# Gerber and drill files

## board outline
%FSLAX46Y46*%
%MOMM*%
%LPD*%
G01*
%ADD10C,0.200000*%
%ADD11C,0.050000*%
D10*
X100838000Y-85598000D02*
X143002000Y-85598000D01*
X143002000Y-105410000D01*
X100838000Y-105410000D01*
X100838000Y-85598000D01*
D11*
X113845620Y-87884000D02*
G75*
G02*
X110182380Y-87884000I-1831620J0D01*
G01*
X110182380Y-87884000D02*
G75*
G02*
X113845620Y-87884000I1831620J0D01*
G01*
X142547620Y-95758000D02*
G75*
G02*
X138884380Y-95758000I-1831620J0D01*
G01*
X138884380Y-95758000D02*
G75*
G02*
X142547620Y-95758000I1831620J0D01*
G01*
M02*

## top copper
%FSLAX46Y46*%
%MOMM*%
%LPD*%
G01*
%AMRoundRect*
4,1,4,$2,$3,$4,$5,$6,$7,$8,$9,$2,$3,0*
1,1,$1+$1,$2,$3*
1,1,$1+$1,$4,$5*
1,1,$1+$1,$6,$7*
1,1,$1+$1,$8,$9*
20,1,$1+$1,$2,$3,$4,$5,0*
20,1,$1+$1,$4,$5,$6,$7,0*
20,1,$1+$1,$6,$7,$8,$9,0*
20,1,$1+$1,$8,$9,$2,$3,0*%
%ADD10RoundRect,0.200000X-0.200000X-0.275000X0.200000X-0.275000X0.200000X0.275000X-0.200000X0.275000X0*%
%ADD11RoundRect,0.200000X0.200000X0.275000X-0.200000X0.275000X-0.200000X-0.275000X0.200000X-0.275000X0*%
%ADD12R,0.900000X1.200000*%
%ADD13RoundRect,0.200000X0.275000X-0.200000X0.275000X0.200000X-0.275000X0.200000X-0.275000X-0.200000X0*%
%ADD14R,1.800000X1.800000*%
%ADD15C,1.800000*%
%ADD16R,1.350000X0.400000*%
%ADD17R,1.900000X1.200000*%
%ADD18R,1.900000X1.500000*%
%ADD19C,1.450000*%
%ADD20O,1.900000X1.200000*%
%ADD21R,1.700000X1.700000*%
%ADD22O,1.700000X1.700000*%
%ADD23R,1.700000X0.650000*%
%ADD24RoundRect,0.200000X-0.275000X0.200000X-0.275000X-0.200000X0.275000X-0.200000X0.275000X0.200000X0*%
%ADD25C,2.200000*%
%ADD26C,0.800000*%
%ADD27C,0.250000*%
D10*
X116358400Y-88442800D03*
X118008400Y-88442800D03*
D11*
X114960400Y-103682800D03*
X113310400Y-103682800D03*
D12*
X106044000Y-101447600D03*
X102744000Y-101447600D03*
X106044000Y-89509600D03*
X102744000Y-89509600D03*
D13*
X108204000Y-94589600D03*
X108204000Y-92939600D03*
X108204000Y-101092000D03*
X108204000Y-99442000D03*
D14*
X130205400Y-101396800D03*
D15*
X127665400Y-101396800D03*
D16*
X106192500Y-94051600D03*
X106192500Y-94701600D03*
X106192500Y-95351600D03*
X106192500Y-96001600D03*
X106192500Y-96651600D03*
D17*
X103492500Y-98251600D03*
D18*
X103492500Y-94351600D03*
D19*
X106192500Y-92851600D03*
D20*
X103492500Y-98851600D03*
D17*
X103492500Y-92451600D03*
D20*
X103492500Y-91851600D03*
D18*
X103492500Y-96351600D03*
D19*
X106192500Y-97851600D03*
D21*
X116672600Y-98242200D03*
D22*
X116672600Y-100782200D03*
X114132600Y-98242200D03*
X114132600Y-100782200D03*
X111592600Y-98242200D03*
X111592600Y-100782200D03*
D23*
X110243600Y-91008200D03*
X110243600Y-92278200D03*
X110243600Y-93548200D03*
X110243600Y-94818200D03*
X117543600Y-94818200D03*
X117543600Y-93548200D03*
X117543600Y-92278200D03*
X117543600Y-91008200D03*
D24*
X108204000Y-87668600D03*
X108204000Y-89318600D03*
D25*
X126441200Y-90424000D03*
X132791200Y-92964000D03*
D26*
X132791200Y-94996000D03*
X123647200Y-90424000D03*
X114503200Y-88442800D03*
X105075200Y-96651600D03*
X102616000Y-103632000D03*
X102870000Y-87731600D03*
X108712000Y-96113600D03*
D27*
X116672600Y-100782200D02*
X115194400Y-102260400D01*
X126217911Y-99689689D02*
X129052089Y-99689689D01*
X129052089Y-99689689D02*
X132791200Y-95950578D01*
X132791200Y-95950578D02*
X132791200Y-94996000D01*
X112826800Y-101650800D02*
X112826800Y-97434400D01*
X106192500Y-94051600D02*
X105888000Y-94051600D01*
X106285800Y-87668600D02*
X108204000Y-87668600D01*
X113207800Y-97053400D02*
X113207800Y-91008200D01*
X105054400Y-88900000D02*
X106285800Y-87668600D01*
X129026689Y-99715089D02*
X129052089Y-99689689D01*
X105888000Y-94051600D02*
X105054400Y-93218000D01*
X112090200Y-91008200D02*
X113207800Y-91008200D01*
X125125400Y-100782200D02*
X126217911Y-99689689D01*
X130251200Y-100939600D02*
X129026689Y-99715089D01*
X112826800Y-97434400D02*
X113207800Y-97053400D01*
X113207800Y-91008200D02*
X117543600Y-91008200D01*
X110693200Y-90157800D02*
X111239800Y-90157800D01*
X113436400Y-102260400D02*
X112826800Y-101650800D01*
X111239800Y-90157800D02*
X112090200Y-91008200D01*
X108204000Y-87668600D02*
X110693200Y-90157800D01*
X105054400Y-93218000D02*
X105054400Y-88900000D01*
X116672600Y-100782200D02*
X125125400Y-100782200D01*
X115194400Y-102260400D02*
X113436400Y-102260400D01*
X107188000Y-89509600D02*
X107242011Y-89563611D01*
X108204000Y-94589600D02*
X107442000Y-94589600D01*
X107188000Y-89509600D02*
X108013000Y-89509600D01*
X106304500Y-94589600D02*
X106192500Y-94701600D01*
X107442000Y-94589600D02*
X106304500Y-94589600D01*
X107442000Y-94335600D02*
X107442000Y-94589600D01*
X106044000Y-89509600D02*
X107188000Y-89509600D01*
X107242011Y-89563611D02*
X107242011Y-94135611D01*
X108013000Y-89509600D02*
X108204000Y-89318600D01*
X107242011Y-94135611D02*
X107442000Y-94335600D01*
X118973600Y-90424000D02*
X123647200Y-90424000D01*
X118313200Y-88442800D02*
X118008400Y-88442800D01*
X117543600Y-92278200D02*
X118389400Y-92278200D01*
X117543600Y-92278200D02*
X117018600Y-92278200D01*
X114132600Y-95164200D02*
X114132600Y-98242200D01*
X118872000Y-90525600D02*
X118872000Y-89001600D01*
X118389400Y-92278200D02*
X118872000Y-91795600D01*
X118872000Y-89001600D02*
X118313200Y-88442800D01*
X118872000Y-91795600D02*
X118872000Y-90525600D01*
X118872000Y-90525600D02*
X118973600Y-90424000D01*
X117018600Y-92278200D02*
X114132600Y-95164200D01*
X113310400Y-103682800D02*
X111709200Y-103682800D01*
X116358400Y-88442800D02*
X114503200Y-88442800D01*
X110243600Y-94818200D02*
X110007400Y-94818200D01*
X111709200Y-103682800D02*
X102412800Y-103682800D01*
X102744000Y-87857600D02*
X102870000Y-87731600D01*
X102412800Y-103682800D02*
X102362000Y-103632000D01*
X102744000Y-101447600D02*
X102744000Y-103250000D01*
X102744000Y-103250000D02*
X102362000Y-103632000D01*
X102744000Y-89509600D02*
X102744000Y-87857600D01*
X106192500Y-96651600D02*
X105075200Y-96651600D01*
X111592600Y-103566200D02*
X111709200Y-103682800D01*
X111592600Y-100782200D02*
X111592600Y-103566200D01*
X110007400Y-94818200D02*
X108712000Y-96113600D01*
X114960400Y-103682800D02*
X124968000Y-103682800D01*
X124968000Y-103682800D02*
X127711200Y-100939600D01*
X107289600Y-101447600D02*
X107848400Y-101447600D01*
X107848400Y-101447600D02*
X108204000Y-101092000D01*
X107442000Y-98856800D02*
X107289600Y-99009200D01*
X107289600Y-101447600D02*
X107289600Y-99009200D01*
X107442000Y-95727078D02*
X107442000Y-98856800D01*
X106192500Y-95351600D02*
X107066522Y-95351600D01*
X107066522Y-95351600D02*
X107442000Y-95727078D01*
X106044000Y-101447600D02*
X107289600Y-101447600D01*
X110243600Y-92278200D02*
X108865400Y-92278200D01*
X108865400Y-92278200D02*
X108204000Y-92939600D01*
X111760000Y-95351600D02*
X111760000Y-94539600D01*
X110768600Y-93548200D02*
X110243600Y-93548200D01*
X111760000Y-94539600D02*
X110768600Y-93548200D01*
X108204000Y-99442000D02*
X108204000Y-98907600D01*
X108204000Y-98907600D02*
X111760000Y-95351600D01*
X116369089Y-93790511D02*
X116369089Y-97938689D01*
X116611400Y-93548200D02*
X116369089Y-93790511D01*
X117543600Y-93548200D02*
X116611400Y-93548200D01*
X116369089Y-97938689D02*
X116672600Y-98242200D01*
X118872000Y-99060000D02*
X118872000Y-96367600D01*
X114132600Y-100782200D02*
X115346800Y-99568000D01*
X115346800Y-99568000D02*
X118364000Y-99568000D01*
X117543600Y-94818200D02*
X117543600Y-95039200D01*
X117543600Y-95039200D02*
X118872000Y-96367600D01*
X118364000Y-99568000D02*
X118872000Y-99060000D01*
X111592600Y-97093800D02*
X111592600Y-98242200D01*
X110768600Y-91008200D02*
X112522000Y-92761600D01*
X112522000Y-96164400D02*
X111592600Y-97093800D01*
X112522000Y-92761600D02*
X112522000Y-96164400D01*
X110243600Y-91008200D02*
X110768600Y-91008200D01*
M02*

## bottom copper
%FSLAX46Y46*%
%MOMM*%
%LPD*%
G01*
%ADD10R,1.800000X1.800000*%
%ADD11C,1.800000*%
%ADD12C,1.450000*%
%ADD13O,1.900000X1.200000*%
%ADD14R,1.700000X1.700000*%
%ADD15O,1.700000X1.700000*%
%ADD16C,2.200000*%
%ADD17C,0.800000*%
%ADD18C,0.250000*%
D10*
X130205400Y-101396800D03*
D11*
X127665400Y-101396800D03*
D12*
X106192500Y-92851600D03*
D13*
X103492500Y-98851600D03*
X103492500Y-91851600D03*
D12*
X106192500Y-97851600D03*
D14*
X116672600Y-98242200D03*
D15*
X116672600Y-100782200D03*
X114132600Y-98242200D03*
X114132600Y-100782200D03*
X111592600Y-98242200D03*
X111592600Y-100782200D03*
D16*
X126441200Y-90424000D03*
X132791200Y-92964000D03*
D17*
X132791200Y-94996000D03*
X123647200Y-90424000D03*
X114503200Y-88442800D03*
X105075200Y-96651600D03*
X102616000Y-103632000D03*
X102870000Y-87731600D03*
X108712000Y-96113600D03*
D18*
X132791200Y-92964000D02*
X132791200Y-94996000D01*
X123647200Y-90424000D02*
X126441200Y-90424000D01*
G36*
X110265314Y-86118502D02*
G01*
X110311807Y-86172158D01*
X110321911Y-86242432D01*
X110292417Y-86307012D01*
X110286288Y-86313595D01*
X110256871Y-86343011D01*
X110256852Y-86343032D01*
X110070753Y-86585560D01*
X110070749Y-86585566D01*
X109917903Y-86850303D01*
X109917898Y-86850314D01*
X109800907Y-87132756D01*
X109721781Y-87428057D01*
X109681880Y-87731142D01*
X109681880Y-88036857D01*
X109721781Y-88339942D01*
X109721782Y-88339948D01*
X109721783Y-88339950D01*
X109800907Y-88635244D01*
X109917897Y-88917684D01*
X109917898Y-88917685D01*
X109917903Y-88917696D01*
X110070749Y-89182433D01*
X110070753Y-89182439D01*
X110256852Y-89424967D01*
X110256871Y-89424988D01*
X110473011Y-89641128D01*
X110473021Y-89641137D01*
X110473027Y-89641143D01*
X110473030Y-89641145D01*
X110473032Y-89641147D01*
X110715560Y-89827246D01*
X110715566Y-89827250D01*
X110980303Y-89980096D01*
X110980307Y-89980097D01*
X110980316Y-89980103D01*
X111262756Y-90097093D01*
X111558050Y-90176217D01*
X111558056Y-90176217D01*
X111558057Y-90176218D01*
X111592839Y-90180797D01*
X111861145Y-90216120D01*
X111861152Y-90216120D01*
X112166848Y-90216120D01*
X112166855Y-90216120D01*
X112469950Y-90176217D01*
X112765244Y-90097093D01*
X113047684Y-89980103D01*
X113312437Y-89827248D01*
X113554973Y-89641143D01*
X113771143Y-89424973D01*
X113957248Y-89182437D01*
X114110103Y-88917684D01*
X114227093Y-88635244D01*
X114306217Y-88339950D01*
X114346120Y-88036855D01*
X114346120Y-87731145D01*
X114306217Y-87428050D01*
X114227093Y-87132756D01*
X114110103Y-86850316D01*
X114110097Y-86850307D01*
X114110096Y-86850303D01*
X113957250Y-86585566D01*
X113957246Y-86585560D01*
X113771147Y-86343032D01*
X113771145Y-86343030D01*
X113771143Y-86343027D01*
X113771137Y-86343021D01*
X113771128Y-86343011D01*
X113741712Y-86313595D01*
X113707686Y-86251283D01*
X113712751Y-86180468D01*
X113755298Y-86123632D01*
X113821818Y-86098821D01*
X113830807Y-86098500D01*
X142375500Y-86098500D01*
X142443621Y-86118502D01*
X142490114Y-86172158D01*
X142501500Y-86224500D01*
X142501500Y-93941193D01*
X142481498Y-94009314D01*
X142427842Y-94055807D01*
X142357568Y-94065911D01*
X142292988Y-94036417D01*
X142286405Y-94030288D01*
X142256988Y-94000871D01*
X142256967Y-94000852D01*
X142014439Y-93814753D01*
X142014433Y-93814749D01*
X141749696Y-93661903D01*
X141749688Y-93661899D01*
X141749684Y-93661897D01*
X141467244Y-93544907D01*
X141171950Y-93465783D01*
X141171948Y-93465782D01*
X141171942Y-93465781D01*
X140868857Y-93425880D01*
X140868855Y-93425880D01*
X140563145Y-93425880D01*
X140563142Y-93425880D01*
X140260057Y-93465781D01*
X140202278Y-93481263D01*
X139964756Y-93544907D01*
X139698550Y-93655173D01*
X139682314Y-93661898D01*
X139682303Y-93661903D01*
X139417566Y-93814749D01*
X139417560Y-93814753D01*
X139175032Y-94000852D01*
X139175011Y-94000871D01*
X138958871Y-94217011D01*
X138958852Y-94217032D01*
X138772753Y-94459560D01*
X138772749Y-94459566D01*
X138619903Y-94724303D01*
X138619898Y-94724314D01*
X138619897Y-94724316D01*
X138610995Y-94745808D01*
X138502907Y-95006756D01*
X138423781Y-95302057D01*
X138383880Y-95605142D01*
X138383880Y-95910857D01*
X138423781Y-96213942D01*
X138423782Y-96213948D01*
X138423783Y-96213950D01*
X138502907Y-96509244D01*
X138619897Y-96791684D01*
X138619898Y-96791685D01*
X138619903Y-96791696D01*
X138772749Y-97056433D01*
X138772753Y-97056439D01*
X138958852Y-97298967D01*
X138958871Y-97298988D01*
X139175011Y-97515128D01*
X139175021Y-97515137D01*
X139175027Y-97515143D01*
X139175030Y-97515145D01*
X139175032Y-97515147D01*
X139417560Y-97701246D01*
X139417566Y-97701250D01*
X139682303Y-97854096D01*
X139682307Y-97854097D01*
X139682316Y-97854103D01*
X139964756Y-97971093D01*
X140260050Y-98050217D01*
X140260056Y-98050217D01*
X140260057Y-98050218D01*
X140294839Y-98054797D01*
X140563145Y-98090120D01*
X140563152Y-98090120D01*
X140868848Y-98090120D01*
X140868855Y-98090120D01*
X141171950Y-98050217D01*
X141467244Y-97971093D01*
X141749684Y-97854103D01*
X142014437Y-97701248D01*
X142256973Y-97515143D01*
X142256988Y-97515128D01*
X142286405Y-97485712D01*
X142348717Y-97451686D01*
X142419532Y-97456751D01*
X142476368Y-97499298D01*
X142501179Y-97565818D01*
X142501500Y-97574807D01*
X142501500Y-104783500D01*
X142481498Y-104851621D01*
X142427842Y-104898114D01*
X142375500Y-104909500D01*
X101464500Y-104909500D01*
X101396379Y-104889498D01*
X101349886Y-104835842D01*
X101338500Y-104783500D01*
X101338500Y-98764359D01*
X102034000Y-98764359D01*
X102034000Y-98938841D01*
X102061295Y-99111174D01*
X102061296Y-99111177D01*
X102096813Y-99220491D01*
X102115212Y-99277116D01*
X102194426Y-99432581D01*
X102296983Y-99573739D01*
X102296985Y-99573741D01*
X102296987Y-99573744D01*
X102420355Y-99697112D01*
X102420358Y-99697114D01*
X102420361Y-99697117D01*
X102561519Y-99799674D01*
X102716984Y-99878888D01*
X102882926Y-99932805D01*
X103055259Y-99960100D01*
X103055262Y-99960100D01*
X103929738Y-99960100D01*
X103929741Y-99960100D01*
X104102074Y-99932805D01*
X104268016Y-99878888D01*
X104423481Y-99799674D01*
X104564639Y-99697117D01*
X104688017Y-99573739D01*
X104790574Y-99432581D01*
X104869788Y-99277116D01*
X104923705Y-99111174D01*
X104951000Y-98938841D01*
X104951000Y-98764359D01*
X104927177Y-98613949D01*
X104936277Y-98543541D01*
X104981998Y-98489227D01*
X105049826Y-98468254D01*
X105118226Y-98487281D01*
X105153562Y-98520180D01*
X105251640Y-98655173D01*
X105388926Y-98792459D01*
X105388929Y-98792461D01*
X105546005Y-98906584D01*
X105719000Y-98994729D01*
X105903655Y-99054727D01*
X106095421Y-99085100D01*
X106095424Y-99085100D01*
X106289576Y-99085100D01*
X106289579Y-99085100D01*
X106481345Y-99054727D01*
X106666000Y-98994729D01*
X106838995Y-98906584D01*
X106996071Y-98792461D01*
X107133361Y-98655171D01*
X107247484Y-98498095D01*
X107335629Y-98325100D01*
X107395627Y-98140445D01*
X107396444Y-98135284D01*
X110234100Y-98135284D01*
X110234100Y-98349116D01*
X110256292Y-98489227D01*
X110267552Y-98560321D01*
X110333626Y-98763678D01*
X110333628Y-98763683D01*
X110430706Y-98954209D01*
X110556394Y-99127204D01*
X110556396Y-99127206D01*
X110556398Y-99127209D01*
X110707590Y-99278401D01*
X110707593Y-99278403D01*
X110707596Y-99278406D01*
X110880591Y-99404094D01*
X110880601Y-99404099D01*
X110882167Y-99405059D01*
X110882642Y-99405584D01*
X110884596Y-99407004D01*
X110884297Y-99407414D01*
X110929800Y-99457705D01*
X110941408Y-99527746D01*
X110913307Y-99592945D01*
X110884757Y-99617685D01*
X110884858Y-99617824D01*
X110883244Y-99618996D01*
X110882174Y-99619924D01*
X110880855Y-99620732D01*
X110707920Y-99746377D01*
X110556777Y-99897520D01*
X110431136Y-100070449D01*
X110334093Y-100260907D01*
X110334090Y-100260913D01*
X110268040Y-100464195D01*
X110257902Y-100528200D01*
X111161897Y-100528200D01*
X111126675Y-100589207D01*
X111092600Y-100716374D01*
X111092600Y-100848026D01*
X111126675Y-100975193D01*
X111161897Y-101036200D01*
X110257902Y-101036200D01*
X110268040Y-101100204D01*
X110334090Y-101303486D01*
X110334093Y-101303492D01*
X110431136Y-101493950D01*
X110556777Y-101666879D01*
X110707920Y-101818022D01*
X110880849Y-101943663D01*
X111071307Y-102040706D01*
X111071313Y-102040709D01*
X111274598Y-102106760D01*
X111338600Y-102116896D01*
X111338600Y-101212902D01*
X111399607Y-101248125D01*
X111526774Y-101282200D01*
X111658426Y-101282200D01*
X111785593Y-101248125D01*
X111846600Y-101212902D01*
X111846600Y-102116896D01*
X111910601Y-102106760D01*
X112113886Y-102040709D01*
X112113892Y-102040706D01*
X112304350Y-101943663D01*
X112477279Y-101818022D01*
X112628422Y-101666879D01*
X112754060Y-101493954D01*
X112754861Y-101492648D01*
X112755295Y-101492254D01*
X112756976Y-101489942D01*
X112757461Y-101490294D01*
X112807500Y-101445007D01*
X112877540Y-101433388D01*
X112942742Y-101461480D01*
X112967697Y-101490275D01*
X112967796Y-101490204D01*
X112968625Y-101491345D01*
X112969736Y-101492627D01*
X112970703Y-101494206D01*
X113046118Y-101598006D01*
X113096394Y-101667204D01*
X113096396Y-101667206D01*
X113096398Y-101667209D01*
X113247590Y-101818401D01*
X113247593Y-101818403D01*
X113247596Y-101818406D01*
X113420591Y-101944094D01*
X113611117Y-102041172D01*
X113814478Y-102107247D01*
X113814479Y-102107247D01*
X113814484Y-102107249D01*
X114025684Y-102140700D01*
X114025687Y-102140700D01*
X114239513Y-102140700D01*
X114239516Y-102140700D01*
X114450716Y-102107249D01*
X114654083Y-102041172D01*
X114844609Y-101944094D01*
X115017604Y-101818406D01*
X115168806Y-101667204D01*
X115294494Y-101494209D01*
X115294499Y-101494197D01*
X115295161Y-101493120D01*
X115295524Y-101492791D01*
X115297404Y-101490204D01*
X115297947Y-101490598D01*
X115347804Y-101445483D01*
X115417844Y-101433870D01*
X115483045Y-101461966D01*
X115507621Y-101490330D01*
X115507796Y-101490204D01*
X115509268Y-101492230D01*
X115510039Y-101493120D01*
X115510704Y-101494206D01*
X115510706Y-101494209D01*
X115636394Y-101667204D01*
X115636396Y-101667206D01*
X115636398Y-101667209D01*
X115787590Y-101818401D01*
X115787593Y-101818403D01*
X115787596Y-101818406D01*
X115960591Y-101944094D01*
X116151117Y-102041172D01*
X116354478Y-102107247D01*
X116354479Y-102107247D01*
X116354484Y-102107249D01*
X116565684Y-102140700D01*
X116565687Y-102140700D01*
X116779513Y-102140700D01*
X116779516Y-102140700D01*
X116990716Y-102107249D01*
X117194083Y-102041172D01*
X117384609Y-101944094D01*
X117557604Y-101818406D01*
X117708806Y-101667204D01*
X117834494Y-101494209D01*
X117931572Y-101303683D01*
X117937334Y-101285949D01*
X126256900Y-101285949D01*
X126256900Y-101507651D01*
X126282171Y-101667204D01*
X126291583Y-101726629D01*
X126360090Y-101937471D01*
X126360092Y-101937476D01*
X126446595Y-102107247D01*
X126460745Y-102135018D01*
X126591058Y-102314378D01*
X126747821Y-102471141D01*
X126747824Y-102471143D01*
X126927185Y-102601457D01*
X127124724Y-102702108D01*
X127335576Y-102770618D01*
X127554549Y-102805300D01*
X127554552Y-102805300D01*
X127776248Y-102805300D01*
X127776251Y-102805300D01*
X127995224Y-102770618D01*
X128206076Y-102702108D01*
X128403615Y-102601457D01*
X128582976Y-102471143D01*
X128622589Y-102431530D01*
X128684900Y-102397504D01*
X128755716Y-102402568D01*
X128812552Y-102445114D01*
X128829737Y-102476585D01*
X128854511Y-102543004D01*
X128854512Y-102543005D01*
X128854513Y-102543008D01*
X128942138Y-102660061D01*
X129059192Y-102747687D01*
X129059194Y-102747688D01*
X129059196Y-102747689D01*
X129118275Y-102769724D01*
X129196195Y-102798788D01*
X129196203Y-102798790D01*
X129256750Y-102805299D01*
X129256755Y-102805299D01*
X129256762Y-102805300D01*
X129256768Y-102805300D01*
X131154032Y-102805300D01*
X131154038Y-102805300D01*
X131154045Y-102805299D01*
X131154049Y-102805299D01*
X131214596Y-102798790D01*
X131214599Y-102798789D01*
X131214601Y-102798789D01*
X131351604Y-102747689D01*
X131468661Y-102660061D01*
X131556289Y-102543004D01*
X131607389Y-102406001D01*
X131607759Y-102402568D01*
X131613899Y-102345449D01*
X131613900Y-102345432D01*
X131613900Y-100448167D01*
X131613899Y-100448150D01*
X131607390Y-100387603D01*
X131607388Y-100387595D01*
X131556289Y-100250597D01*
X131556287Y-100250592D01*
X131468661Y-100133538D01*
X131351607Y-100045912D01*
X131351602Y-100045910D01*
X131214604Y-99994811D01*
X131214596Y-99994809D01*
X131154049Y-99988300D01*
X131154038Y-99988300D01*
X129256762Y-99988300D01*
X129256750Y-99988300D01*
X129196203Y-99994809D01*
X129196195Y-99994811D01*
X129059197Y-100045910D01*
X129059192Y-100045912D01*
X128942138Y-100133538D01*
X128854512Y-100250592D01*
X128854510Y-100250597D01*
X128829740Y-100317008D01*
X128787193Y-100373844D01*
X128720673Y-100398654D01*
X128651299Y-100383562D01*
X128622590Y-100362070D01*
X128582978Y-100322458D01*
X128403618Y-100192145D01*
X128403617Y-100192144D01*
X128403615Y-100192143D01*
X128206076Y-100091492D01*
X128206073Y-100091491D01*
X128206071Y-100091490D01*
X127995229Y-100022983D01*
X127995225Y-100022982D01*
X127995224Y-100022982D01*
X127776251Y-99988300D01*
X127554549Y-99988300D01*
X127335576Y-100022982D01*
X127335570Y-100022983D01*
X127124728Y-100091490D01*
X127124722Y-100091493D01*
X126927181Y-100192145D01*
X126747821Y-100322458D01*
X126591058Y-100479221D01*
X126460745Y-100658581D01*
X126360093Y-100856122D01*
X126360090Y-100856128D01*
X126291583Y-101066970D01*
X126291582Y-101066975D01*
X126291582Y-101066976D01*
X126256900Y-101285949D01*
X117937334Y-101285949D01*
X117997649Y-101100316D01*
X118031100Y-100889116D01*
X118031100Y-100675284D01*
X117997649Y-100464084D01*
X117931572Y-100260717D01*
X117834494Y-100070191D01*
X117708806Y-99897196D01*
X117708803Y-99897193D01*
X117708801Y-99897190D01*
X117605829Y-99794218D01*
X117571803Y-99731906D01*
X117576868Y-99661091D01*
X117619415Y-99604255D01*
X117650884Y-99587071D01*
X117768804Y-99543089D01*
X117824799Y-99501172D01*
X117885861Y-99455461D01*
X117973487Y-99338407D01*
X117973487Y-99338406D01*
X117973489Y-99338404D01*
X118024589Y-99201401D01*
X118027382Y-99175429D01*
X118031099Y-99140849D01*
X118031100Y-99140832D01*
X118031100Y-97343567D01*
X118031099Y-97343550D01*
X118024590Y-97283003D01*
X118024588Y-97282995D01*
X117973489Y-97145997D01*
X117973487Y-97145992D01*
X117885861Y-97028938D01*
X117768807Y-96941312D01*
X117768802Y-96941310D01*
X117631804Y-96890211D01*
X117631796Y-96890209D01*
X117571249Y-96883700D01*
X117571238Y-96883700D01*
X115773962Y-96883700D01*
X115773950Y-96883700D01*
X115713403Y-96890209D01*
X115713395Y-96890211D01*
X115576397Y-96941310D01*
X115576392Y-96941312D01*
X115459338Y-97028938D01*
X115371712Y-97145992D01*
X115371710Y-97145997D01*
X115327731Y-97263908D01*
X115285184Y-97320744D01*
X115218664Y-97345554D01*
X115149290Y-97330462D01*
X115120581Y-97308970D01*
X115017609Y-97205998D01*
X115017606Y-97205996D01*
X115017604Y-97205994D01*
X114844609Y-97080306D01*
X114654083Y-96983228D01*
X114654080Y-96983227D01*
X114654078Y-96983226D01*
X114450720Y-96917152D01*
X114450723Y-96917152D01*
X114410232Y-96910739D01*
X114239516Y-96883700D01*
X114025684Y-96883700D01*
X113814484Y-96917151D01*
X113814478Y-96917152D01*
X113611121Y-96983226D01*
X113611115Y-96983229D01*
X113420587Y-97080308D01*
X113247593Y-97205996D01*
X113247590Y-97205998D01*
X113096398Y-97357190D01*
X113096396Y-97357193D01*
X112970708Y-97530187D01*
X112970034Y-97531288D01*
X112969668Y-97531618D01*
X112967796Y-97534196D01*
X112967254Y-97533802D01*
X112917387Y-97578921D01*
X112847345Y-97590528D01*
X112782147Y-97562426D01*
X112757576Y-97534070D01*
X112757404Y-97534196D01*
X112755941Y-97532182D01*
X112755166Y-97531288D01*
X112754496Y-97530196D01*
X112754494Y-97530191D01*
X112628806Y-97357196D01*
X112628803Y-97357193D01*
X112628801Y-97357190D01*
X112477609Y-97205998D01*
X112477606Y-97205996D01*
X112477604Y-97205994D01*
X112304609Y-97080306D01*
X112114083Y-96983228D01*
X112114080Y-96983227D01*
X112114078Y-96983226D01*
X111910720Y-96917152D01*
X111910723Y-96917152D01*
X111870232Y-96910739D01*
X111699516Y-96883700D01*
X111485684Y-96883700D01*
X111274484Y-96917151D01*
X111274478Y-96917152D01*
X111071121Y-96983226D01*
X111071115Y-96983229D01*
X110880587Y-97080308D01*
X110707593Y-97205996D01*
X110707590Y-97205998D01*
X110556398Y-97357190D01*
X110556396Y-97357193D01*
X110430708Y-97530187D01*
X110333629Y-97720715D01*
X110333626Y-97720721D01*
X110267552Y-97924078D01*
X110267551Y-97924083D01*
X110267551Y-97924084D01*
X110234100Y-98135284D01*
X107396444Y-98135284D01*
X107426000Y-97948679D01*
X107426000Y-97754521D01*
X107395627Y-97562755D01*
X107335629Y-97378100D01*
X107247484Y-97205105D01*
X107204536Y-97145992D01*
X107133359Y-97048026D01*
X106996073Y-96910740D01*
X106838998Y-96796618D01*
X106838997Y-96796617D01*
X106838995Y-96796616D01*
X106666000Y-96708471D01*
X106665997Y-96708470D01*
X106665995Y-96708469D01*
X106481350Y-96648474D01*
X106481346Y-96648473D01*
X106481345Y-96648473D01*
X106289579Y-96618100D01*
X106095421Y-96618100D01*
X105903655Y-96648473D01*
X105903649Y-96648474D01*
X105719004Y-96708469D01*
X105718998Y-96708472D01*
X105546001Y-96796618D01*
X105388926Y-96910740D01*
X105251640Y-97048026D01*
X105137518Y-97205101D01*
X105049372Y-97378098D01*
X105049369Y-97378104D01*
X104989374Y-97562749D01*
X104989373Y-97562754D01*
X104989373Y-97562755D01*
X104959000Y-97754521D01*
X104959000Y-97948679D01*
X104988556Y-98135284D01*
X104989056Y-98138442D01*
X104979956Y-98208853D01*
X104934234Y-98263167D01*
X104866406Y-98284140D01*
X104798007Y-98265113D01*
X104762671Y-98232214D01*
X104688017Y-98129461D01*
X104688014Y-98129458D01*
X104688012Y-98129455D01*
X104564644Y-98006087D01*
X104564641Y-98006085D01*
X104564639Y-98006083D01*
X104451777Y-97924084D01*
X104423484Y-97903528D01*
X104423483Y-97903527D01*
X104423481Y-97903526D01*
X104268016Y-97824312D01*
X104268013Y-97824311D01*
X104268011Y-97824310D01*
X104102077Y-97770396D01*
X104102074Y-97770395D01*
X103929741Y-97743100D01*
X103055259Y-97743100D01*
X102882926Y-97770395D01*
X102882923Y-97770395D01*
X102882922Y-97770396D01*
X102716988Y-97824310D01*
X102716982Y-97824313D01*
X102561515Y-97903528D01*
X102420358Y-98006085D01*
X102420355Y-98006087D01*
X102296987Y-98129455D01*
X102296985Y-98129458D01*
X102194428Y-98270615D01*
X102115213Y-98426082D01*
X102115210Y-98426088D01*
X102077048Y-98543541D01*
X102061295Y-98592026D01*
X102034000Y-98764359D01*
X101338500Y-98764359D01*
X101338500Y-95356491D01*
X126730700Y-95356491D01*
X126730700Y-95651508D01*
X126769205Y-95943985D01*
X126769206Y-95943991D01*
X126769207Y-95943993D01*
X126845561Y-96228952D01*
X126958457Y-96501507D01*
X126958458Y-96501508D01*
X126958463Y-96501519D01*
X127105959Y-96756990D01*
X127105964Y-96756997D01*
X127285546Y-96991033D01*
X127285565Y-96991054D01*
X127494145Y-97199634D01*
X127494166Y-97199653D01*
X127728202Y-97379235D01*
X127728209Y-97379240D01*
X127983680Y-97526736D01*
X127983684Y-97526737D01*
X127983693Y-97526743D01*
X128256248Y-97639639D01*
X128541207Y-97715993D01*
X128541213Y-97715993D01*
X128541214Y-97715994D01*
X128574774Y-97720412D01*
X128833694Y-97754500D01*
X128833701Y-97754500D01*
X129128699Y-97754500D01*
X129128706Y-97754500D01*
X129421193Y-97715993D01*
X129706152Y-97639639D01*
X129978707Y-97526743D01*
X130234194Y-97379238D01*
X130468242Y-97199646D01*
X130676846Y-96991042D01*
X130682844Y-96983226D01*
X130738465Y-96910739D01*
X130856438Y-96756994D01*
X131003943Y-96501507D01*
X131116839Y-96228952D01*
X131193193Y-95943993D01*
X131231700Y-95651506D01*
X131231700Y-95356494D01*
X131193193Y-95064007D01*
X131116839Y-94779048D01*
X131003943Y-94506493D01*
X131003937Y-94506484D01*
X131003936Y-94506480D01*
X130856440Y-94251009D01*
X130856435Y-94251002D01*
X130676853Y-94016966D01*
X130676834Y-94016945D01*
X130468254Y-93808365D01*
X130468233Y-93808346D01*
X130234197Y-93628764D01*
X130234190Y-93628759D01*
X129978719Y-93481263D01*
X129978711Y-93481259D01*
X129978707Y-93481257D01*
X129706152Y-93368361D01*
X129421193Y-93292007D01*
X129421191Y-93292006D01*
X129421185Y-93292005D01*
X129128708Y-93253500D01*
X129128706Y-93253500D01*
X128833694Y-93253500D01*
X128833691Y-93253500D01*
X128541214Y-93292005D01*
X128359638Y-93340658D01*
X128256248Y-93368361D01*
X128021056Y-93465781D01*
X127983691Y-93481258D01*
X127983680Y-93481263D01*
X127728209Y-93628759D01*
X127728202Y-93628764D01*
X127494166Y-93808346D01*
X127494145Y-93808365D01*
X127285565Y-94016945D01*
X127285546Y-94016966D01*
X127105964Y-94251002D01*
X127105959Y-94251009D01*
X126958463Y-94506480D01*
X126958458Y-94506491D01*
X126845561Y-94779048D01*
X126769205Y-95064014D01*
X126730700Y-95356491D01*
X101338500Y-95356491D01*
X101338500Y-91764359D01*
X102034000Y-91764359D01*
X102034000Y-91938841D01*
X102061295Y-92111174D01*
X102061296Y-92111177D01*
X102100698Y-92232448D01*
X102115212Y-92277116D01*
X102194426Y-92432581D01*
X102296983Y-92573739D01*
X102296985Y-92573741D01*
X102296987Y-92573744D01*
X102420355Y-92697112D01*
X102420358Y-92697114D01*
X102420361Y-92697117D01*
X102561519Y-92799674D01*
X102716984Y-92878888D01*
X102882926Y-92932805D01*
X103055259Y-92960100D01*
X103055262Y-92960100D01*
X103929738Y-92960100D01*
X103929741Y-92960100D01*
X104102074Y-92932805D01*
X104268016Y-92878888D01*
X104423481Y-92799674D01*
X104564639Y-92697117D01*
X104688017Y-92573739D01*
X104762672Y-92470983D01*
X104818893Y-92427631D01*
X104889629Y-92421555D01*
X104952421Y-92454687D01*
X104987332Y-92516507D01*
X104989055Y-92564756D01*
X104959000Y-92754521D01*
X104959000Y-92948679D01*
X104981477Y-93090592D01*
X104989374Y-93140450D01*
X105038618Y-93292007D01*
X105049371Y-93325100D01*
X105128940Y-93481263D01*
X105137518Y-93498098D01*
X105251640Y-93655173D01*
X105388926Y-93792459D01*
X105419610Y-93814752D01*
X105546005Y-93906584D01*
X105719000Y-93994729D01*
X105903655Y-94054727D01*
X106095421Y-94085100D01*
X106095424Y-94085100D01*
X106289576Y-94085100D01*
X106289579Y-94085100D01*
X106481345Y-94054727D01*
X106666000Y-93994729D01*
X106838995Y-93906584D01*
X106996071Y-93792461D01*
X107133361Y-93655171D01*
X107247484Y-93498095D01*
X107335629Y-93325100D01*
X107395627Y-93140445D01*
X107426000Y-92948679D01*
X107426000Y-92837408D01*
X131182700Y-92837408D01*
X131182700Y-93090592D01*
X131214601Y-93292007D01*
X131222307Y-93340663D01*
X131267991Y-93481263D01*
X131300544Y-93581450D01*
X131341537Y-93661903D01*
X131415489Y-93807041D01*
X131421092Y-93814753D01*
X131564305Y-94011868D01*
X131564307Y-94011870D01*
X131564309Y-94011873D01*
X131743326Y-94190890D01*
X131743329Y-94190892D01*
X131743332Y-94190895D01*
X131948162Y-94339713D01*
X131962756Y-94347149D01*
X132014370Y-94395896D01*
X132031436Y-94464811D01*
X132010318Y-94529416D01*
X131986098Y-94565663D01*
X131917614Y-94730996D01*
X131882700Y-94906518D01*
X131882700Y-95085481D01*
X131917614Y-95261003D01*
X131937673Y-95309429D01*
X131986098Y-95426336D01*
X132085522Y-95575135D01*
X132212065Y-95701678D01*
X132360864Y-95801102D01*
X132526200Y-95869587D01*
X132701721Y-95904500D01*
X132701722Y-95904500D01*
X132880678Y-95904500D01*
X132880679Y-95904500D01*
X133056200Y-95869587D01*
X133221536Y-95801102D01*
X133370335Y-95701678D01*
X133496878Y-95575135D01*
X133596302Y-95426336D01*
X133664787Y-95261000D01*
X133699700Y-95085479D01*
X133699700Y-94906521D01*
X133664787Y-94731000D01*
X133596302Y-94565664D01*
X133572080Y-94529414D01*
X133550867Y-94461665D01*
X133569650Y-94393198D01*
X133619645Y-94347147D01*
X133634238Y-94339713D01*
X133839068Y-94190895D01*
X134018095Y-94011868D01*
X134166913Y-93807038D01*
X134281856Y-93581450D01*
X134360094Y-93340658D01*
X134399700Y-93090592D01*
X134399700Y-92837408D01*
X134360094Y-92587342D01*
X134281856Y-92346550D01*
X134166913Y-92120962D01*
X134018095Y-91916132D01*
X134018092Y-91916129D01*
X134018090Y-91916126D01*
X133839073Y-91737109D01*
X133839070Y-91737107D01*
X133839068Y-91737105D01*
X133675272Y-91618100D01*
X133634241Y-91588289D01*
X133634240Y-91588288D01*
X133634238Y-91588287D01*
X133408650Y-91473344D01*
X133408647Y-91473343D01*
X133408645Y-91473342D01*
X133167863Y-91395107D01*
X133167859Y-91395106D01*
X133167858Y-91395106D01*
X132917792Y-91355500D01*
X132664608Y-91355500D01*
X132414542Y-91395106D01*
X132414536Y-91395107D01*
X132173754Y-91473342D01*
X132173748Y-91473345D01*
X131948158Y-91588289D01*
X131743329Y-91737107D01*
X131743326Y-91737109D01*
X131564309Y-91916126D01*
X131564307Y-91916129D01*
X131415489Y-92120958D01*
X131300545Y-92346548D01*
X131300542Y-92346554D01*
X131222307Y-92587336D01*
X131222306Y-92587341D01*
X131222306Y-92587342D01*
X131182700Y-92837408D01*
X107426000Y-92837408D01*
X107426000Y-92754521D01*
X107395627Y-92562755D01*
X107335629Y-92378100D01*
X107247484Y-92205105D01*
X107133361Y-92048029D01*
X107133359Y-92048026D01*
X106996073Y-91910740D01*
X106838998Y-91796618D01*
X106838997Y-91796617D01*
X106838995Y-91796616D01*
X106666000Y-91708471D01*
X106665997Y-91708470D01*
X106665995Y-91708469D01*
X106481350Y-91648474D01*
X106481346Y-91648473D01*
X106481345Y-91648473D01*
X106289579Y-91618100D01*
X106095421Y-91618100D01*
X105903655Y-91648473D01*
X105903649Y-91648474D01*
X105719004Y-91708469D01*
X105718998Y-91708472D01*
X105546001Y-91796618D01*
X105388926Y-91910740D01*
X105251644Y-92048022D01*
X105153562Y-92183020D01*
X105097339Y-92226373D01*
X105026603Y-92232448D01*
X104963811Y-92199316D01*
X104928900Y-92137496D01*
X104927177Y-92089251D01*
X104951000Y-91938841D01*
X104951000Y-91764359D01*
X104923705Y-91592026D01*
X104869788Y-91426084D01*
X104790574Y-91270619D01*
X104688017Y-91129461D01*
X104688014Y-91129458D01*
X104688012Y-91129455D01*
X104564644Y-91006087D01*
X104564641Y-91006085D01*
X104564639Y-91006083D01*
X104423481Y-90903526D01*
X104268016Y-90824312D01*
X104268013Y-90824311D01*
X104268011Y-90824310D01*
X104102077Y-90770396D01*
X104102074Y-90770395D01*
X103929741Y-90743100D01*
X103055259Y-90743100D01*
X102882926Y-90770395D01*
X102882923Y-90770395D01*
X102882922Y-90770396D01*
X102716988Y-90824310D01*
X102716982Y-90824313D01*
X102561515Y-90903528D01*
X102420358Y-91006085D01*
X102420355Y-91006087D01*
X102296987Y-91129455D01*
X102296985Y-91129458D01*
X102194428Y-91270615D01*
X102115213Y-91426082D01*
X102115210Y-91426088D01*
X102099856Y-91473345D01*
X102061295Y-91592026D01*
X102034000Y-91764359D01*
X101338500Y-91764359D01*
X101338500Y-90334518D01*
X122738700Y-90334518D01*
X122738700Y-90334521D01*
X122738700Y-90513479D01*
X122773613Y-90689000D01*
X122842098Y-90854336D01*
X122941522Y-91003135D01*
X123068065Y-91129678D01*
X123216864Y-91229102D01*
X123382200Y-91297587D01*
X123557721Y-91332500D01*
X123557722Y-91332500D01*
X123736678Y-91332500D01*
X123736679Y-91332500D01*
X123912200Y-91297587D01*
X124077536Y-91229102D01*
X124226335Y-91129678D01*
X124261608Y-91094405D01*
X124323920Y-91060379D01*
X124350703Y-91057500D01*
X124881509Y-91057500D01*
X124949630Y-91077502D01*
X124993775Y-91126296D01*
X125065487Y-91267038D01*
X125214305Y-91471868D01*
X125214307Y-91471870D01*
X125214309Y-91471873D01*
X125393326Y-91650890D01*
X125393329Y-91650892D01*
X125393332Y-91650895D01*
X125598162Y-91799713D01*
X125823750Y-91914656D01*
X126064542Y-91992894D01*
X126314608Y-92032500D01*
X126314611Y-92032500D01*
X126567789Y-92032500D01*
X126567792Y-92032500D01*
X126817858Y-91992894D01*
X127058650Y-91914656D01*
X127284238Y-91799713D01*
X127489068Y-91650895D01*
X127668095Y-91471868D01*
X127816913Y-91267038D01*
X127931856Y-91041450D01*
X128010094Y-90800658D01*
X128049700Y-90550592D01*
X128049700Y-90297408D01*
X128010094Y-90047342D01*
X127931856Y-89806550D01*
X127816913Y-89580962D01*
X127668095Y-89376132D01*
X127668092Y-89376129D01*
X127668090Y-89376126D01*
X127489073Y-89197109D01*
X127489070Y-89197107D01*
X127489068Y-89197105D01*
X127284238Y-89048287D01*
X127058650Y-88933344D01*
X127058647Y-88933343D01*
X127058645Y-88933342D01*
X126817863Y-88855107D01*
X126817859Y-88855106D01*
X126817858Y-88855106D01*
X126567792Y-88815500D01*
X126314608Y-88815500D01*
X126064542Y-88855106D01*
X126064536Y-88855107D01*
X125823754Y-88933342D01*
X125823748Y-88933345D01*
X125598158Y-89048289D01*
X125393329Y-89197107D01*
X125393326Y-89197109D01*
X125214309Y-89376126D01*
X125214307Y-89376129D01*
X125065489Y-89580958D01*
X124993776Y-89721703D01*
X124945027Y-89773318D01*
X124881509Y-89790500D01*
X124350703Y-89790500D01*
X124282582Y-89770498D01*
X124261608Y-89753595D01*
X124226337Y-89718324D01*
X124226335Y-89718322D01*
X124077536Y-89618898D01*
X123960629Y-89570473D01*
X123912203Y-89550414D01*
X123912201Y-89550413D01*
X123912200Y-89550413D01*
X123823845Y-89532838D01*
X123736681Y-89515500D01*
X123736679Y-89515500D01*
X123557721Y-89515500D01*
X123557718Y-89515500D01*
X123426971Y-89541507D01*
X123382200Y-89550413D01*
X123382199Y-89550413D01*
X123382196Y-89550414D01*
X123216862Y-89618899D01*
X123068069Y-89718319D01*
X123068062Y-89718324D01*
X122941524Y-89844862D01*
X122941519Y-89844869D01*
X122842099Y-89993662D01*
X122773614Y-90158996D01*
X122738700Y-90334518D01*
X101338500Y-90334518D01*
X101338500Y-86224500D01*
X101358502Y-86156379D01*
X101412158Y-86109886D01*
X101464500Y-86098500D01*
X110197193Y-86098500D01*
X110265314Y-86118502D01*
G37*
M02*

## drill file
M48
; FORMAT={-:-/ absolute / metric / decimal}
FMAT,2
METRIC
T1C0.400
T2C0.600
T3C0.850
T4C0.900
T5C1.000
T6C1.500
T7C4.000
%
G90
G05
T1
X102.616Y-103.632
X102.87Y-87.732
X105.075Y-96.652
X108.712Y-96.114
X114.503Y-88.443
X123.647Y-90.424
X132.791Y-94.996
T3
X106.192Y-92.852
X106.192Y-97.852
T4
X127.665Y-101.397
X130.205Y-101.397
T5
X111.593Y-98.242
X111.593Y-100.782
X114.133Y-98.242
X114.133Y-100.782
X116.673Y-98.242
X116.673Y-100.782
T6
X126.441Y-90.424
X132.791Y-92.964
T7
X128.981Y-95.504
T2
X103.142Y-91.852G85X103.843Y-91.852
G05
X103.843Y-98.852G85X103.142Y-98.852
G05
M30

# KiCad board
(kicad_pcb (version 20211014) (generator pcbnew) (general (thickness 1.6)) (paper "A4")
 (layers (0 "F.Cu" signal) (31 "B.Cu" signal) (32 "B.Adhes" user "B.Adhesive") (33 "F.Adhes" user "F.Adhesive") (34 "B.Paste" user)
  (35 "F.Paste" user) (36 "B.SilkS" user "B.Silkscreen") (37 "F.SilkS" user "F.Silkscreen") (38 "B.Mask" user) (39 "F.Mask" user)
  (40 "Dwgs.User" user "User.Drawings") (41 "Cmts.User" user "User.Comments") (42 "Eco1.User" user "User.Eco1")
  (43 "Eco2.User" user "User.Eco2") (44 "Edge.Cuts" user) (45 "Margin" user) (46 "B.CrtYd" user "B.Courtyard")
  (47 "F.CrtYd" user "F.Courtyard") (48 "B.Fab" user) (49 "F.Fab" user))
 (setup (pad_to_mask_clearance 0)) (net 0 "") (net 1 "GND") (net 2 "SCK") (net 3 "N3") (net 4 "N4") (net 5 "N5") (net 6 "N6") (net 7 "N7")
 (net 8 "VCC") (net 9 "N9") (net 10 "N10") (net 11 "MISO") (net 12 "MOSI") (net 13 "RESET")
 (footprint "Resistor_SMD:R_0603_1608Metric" (layer "F.Cu") (at 117.1834 88.4428)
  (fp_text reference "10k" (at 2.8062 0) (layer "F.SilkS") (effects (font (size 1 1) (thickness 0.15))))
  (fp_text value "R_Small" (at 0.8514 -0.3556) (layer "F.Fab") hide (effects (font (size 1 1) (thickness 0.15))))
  (pad "1" smd roundrect locked (at -0.825 0) (size 0.8 0.95) (layers "F.Cu" "F.Paste" "F.Mask") (roundrect_rratio 0.25) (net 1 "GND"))
  (pad "2" smd roundrect locked (at 0.825 0) (size 0.8 0.95) (layers "F.Cu" "F.Paste" "F.Mask") (roundrect_rratio 0.25) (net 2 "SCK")))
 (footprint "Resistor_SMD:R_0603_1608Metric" (layer "F.Cu") (at 114.1354 103.6828 180)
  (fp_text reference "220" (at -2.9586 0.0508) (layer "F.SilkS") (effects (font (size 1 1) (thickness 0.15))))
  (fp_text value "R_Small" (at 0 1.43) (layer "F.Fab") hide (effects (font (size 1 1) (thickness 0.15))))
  (pad "1" smd roundrect locked (at -0.825 0 180) (size 0.8 0.95) (layers "F.Cu" "F.Paste" "F.Mask") (roundrect_rratio 0.25) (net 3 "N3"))
  (pad "2" smd roundrect locked (at 0.825 0 180) (size 0.8 0.95) (layers "F.Cu" "F.Paste" "F.Mask") (roundrect_rratio 0.25) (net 1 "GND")))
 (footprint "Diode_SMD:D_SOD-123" (layer "F.Cu") (at 104.394 101.4476 180)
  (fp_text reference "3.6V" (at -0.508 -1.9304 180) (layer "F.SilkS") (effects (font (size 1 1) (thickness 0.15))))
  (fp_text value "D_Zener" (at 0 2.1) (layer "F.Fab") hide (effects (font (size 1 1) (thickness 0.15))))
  (pad "1" smd rect locked (at -1.65 0 180) (size 0.9 1.2) (layers "F.Cu" "F.Paste" "F.Mask") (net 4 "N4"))
  (pad "2" smd rect locked (at 1.65 0 180) (size 0.9 1.2) (layers "F.Cu" "F.Paste" "F.Mask") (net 1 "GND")))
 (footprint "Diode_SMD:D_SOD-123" (layer "F.Cu") (at 104.394 89.5096 180)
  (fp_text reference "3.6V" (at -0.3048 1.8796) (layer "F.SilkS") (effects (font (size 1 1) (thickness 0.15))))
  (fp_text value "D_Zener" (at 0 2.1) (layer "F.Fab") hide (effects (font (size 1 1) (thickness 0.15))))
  (pad "1" smd rect locked (at -1.65 0 180) (size 0.9 1.2) (layers "F.Cu" "F.Paste" "F.Mask") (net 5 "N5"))
  (pad "2" smd rect locked (at 1.65 0 180) (size 0.9 1.2) (layers "F.Cu" "F.Paste" "F.Mask") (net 1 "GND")))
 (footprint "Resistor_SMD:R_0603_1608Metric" (layer "F.Cu") (at 108.204 93.7646 90)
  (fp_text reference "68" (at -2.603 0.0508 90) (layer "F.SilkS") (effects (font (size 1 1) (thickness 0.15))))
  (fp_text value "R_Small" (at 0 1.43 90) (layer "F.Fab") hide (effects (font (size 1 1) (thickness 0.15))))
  (pad "1" smd roundrect locked (at -0.825 0 90) (size 0.8 0.95) (layers "F.Cu" "F.Paste" "F.Mask") (roundrect_rratio 0.25) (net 5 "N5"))
  (pad "2" smd roundrect locked (at 0.825 0 90) (size 0.8 0.95) (layers "F.Cu" "F.Paste" "F.Mask") (roundrect_rratio 0.25) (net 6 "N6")))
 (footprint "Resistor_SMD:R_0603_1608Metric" (layer "F.Cu") (at 108.204 100.267 90)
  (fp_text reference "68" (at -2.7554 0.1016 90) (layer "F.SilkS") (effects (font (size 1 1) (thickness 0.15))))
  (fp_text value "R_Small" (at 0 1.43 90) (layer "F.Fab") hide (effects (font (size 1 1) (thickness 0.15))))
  (pad "1" smd roundrect locked (at -0.825 0 90) (size 0.8 0.95) (layers "F.Cu" "F.Paste" "F.Mask") (roundrect_rratio 0.25) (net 4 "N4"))
  (pad "2" smd roundrect locked (at 0.825 0 90) (size 0.8 0.95) (layers "F.Cu" "F.Paste" "F.Mask") (roundrect_rratio 0.25) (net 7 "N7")))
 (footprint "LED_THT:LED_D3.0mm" (layer "F.Cu") (at 130.2054 101.3968 180)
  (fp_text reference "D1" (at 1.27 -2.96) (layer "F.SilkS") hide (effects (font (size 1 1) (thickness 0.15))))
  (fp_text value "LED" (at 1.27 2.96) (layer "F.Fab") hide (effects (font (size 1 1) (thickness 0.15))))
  (pad "1" thru_hole rect locked (at 0 0 180) (size 1.8 1.8) (drill 0.9) (layers *.Cu *.Mask) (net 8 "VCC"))
  (pad "2" thru_hole circle locked (at 2.54 0 180) (size 1.8 1.8) (drill 0.9) (layers *.Cu *.Mask) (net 3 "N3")))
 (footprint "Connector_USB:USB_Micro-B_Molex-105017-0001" (layer "F.Cu") (at 104.73 95.3516 -90)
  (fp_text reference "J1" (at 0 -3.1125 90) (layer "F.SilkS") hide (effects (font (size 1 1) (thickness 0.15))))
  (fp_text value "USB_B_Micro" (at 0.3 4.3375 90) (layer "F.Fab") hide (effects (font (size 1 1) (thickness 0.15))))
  (pad "1" smd rect locked (at -1.3 -1.4625 270) (size 0.4 1.35) (layers "F.Cu" "F.Paste" "F.Mask") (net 8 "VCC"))
  (pad "2" smd rect locked (at -0.65 -1.4625 270) (size 0.4 1.35) (layers "F.Cu" "F.Paste" "F.Mask") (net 5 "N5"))
  (pad "3" smd rect locked (at 0 -1.4625 270) (size 0.4 1.35) (layers "F.Cu" "F.Paste" "F.Mask") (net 4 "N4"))
  (pad "4" smd rect locked (at 0.65 -1.4625 270) (size 0.4 1.35) (layers "F.Cu" "F.Paste" "F.Mask") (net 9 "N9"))
  (pad "5" smd rect locked (at 1.3 -1.4625 270) (size 0.4 1.35) (layers "F.Cu" "F.Paste" "F.Mask") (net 1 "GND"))
  (pad "6" smd rect locked (at 2.9 1.2375 270) (size 1.2 1.9) (layers "F.Cu" "F.Mask") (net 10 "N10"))
  (pad "6" smd rect locked (at -1 1.2375 270) (size 1.5 1.9) (layers "F.Cu" "F.Paste" "F.Mask") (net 10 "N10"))
  (pad "6" thru_hole circle locked (at -2.5 -1.4625 270) (size 1.45 1.45) (drill 0.85) (layers *.Cu *.Mask) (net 10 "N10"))
  (pad "6" thru_hole oval locked (at 3.5 1.2375 270) (size 1.2 1.9) (drill oval 0.6 1.3) (layers *.Cu *.Mask) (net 10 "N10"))
  (pad "6" smd rect locked (at -2.9 1.2375 270) (size 1.2 1.9) (layers "F.Cu" "F.Mask") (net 10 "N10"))
  (pad "6" thru_hole oval locked (at -3.5 1.2375 90) (size 1.2 1.9) (drill oval 0.6 1.3) (layers *.Cu *.Mask) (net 10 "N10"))
  (pad "6" smd rect locked (at 1 1.2375 270) (size 1.5 1.9) (layers "F.Cu" "F.Paste" "F.Mask") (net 10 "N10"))
  (pad "6" thru_hole circle locked (at 2.5 -1.4625 270) (size 1.45 1.45) (drill 0.85) (layers *.Cu *.Mask) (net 10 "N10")))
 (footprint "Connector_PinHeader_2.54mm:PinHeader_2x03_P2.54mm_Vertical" (layer "F.Cu") (at 116.6726 98.2422 -90)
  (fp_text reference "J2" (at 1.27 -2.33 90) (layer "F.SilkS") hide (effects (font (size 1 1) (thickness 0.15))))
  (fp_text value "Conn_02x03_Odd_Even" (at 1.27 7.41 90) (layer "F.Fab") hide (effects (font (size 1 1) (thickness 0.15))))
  (pad "1" thru_hole rect locked (at 0 0 270) (size 1.7 1.7) (drill 1) (layers *.Cu *.Mask) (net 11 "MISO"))
  (pad "2" thru_hole oval locked (at 2.54 0 270) (size 1.7 1.7) (drill 1) (layers *.Cu *.Mask) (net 8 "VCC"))
  (pad "3" thru_hole oval locked (at 0 2.54 270) (size 1.7 1.7) (drill 1) (layers *.Cu *.Mask) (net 2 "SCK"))
  (pad "4" thru_hole oval locked (at 2.54 2.54 270) (size 1.7 1.7) (drill 1) (layers *.Cu *.Mask) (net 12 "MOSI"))
  (pad "5" thru_hole oval locked (at 0 5.08 270) (size 1.7 1.7) (drill 1) (layers *.Cu *.Mask) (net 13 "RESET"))
  (pad "6" thru_hole oval locked (at 2.54 5.08 270) (size 1.7 1.7) (drill 1) (layers *.Cu *.Mask) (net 1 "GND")))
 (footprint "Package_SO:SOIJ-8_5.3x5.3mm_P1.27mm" (layer "F.Cu") (at 113.8936 92.9132)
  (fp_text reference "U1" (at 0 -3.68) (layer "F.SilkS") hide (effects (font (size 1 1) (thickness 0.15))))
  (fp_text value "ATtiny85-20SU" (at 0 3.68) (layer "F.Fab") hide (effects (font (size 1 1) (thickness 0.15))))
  (pad "1" smd rect locked (at -3.65 -1.905) (size 1.7 0.65) (layers "F.Cu" "F.Paste" "F.Mask") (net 13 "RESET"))
  (pad "2" smd rect locked (at -3.65 -0.635) (size 1.7 0.65) (layers "F.Cu" "F.Paste" "F.Mask") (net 6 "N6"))
  (pad "3" smd rect locked (at -3.65 0.635) (size 1.7 0.65) (layers "F.Cu" "F.Paste" "F.Mask") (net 7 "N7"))
  (pad "4" smd rect locked (at -3.65 1.905) (size 1.7 0.65) (layers "F.Cu" "F.Paste" "F.Mask") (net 1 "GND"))
  (pad "5" smd rect locked (at 3.65 1.905) (size 1.7 0.65) (layers "F.Cu" "F.Paste" "F.Mask") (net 12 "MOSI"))
  (pad "6" smd rect locked (at 3.65 0.635) (size 1.7 0.65) (layers "F.Cu" "F.Paste" "F.Mask") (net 11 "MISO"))
  (pad "7" smd rect locked (at 3.65 -0.635) (size 1.7 0.65) (layers "F.Cu" "F.Paste" "F.Mask") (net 2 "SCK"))
  (pad "8" smd rect locked (at 3.65 -1.905) (size 1.7 0.65) (layers "F.Cu" "F.Paste" "F.Mask") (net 8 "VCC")))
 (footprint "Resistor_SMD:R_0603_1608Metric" (layer "F.Cu") (at 108.204 88.4936 -90)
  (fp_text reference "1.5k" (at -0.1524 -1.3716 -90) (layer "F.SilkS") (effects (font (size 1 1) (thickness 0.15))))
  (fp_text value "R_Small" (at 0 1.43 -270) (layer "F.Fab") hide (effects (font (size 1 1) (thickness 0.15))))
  (pad "1" smd roundrect locked (at -0.825 0 270) (size 0.8 0.95) (layers "F.Cu" "F.Paste" "F.Mask") (roundrect_rratio 0.25) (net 8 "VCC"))
  (pad "2" smd roundrect locked (at 0.825 0 270) (size 0.8 0.95) (layers "F.Cu" "F.Paste" "F.Mask") (roundrect_rratio 0.25) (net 5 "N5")))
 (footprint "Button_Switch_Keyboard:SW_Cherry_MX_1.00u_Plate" (layer "B.Cu") (at 126.4412 90.424 180)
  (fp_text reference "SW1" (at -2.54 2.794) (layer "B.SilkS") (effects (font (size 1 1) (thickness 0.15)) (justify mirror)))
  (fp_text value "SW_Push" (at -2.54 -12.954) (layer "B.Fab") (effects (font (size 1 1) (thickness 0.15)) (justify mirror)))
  (pad "" np_thru_hole circle locked (at -2.54 -5.08 180) (size 4 4) (drill 4) (layers *.Cu *.Mask))
  (pad "1" thru_hole circle locked (at 0 0 180) (size 2.2 2.2) (drill 1.5) (layers *.Cu *.Mask) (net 2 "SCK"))
  (pad "2" thru_hole circle locked (at -6.35 -2.54 180) (size 2.2 2.2) (drill 1.5) (layers *.Cu *.Mask) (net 8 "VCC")))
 (gr_rect (start 143.002 85.598) (end 100.838 105.41) (layer "Edge.Cuts") (width 0.2) (fill none))
 (gr_circle (center 112.014 87.884) (end 110.49 86.868) (layer "Edge.Cuts") (width 0.05) (fill none))
 (gr_circle (center 140.716 95.758) (end 139.192 94.742) (layer "Edge.Cuts") (width 0.05) (fill none))
 (segment (start 116.6726 100.7822) (end 115.1944 102.2604) (width 0.25) (layer "F.Cu") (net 8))
 (segment (start 126.217911 99.689689) (end 129.052089 99.689689) (width 0.25) (layer "F.Cu") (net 8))
 (segment (start 129.052089 99.689689) (end 132.7912 95.950578) (width 0.25) (layer "F.Cu") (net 8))
 (segment (start 132.7912 95.950578) (end 132.7912 94.996) (width 0.25) (layer "F.Cu") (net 8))
 (segment (start 112.8268 101.6508) (end 112.8268 97.4344) (width 0.25) (layer "F.Cu") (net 8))
 (segment (start 106.1925 94.0516) (end 105.888 94.0516) (width 0.25) (layer "F.Cu") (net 8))
 (segment (start 106.2858 87.6686) (end 108.204 87.6686) (width 0.25) (layer "F.Cu") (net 8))
 (segment (start 113.2078 97.0534) (end 113.2078 91.0082) (width 0.25) (layer "F.Cu") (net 8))
 (segment (start 105.0544 88.9) (end 106.2858 87.6686) (width 0.25) (layer "F.Cu") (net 8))
 (segment (start 129.026689 99.715089) (end 129.052089 99.689689) (width 0.25) (layer "F.Cu") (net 8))
 (segment (start 105.888 94.0516) (end 105.0544 93.218) (width 0.25) (layer "F.Cu") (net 8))
 (segment (start 112.0902 91.0082) (end 113.2078 91.0082) (width 0.25) (layer "F.Cu") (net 8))
 (segment (start 125.1254 100.7822) (end 126.217911 99.689689) (width 0.25) (layer "F.Cu") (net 8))
 (segment (start 130.2512 100.9396) (end 129.026689 99.715089) (width 0.25) (layer "F.Cu") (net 8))
 (segment (start 112.8268 97.4344) (end 113.2078 97.0534) (width 0.25) (layer "F.Cu") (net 8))
 (segment (start 113.2078 91.0082) (end 117.5436 91.0082) (width 0.25) (layer "F.Cu") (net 8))
 (segment (start 110.6932 90.1578) (end 111.2398 90.1578) (width 0.25) (layer "F.Cu") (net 8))
 (segment (start 113.4364 102.2604) (end 112.8268 101.6508) (width 0.25) (layer "F.Cu") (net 8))
 (segment (start 111.2398 90.1578) (end 112.0902 91.0082) (width 0.25) (layer "F.Cu") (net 8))
 (segment (start 108.204 87.6686) (end 110.6932 90.1578) (width 0.25) (layer "F.Cu") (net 8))
 (segment (start 105.0544 93.218) (end 105.0544 88.9) (width 0.25) (layer "F.Cu") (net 8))
 (segment (start 116.6726 100.7822) (end 125.1254 100.7822) (width 0.25) (layer "F.Cu") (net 8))
 (segment (start 115.1944 102.2604) (end 113.4364 102.2604) (width 0.25) (layer "F.Cu") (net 8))
 (via (at 132.7912 94.996) (size 0.8) (drill 0.4) (layers "F.Cu" "B.Cu") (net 8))
 (segment (start 132.7912 92.964) (end 132.7912 94.996) (width 0.25) (layer "B.Cu") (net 8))
 (segment (start 107.188 89.5096) (end 107.242011 89.563611) (width 0.25) (layer "F.Cu") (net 5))
 (segment (start 108.204 94.5896) (end 107.442 94.5896) (width 0.25) (layer "F.Cu") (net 5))
 (segment (start 107.188 89.5096) (end 108.013 89.5096) (width 0.25) (layer "F.Cu") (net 5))
 (segment (start 106.3045 94.5896) (end 106.1925 94.7016) (width 0.25) (layer "F.Cu") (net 5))
 (segment (start 107.442 94.5896) (end 106.3045 94.5896) (width 0.25) (layer "F.Cu") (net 5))
 (segment (start 107.442 94.3356) (end 107.442 94.5896) (width 0.25) (layer "F.Cu") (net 5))
 (segment (start 106.044 89.5096) (end 107.188 89.5096) (width 0.25) (layer "F.Cu") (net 5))
 (segment (start 107.242011 89.563611) (end 107.242011 94.135611) (width 0.25) (layer "F.Cu") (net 5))
 (segment (start 108.013 89.5096) (end 108.204 89.3186) (width 0.25) (layer "F.Cu") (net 5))
 (segment (start 107.242011 94.135611) (end 107.442 94.3356) (width 0.25) (layer "F.Cu") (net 5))
 (segment (start 118.9736 90.424) (end 123.6472 90.424) (width 0.25) (layer "F.Cu") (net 2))
 (segment (start 118.3132 88.4428) (end 118.0084 88.4428) (width 0.25) (layer "F.Cu") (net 2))
 (segment (start 117.5436 92.2782) (end 118.3894 92.2782) (width 0.25) (layer "F.Cu") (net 2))
 (segment (start 117.5436 92.2782) (end 117.0186 92.2782) (width 0.25) (layer "F.Cu") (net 2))
 (segment (start 114.1326 95.1642) (end 114.1326 98.2422) (width 0.25) (layer "F.Cu") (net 2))
 (segment (start 118.872 90.5256) (end 118.872 89.0016) (width 0.25) (layer "F.Cu") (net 2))
 (segment (start 118.3894 92.2782) (end 118.872 91.7956) (width 0.25) (layer "F.Cu") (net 2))
 (segment (start 118.872 89.0016) (end 118.3132 88.4428) (width 0.25) (layer "F.Cu") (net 2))
 (segment (start 118.872 91.7956) (end 118.872 90.5256) (width 0.25) (layer "F.Cu") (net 2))
 (segment (start 118.872 90.5256) (end 118.9736 90.424) (width 0.25) (layer "F.Cu") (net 2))
 (segment (start 117.0186 92.2782) (end 114.1326 95.1642) (width 0.25) (layer "F.Cu") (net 2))
 (via (at 123.6472 90.424) (size 0.8) (drill 0.4) (layers "F.Cu" "B.Cu") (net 2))
 (segment (start 123.6472 90.424) (end 126.4412 90.424) (width 0.25) (layer "B.Cu") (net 2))
 (segment (start 113.3104 103.6828) (end 111.7092 103.6828) (width 0.25) (layer "F.Cu") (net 1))
 (segment (start 116.3584 88.4428) (end 114.5032 88.4428) (width 0.25) (layer "F.Cu") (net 1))
 (segment (start 110.2436 94.8182) (end 110.0074 94.8182) (width 0.25) (layer "F.Cu") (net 1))
 (segment (start 111.7092 103.6828) (end 102.4128 103.6828) (width 0.25) (layer "F.Cu") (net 1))
 (segment (start 102.744 87.8576) (end 102.87 87.7316) (width 0.25) (layer "F.Cu") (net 1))
 (segment (start 102.4128 103.6828) (end 102.362 103.632) (width 0.25) (layer "F.Cu") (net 1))
 (segment (start 102.744 101.4476) (end 102.744 103.25) (width 0.25) (layer "F.Cu") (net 1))
 (segment (start 102.744 103.25) (end 102.362 103.632) (width 0.25) (layer "F.Cu") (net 1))
 (segment (start 102.744 89.5096) (end 102.744 87.8576) (width 0.25) (layer "F.Cu") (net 1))
 (segment (start 106.1925 96.6516) (end 105.0752 96.6516) (width 0.25) (layer "F.Cu") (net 1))
 (segment (start 111.5926 103.5662) (end 111.7092 103.6828) (width 0.25) (layer "F.Cu") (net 1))
 (segment (start 111.5926 100.7822) (end 111.5926 103.5662) (width 0.25) (layer "F.Cu") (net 1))
 (segment (start 110.0074 94.8182) (end 108.712 96.1136) (width 0.25) (layer "F.Cu") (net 1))
 (via (at 114.5032 88.4428) (size 0.8) (drill 0.4) (layers "F.Cu" "B.Cu") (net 1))
 (via (at 105.0752 96.6516) (size 0.8) (drill 0.4) (layers "F.Cu" "B.Cu") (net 1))
 (via (at 102.616 103.632) (size 0.8) (drill 0.4) (layers "F.Cu" "B.Cu") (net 1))
 (via (at 102.87 87.7316) (size 0.8) (drill 0.4) (layers "F.Cu" "B.Cu") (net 1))
 (via (at 108.712 96.1136) (size 0.8) (drill 0.4) (layers "F.Cu" "B.Cu") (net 1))
 (segment (start 114.9604 103.6828) (end 124.968 103.6828) (width 0.25) (layer "F.Cu") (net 3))
 (segment (start 124.968 103.6828) (end 127.7112 100.9396) (width 0.25) (layer "F.Cu") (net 3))
 (segment (start 107.2896 101.4476) (end 107.8484 101.4476) (width 0.25) (layer "F.Cu") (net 4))
 (segment (start 107.8484 101.4476) (end 108.204 101.092) (width 0.25) (layer "F.Cu") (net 4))
 (segment (start 107.442 98.8568) (end 107.2896 99.0092) (width 0.25) (layer "F.Cu") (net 4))
 (segment (start 107.2896 101.4476) (end 107.2896 99.0092) (width 0.25) (layer "F.Cu") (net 4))
 (segment (start 107.442 95.727078) (end 107.442 98.8568) (width 0.25) (layer "F.Cu") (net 4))
 (segment (start 106.1925 95.3516) (end 107.066522 95.3516) (width 0.25) (layer "F.Cu") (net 4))
 (segment (start 107.066522 95.3516) (end 107.442 95.727078) (width 0.25) (layer "F.Cu") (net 4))
 (segment (start 106.044 101.4476) (end 107.2896 101.4476) (width 0.25) (layer "F.Cu") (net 4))
 (segment (start 110.2436 92.2782) (end 108.8654 92.2782) (width 0.25) (layer "F.Cu") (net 6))
 (segment (start 108.8654 92.2782) (end 108.204 92.9396) (width 0.25) (layer "F.Cu") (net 6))
 (segment (start 111.76 95.3516) (end 111.76 94.5396) (width 0.25) (layer "F.Cu") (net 7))
 (segment (start 110.7686 93.5482) (end 110.2436 93.5482) (width 0.25) (layer "F.Cu") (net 7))
 (segment (start 111.76 94.5396) (end 110.7686 93.5482) (width 0.25) (layer "F.Cu") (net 7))
 (segment (start 108.204 99.442) (end 108.204 98.9076) (width 0.25) (layer "F.Cu") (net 7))
 (segment (start 108.204 98.9076) (end 111.76 95.3516) (width 0.25) (layer "F.Cu") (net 7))
 (segment (start 116.369089 93.790511) (end 116.369089 97.938689) (width 0.25) (layer "F.Cu") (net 11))
 (segment (start 116.6114 93.5482) (end 116.369089 93.790511) (width 0.25) (layer "F.Cu") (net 11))
 (segment (start 117.5436 93.5482) (end 116.6114 93.5482) (width 0.25) (layer "F.Cu") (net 11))
 (segment (start 116.369089 97.938689) (end 116.6726 98.2422) (width 0.25) (layer "F.Cu") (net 11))
 (segment (start 118.872 99.06) (end 118.872 96.3676) (width 0.25) (layer "F.Cu") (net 12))
 (segment (start 114.1326 100.7822) (end 115.3468 99.568) (width 0.25) (layer "F.Cu") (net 12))
 (segment (start 115.3468 99.568) (end 118.364 99.568) (width 0.25) (layer "F.Cu") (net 12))
 (segment (start 117.5436 94.8182) (end 117.5436 95.0392) (width 0.25) (layer "F.Cu") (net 12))
 (segment (start 117.5436 95.0392) (end 118.872 96.3676) (width 0.25) (layer "F.Cu") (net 12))
 (segment (start 118.364 99.568) (end 118.872 99.06) (width 0.25) (layer "F.Cu") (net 12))
 (segment (start 111.5926 97.0938) (end 111.5926 98.2422) (width 0.25) (layer "F.Cu") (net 13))
 (segment (start 110.7686 91.0082) (end 112.522 92.7616) (width 0.25) (layer "F.Cu") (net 13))
 (segment (start 112.522 96.1644) (end 111.5926 97.0938) (width 0.25) (layer "F.Cu") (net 13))
 (segment (start 112.522 92.7616) (end 112.522 96.1644) (width 0.25) (layer "F.Cu") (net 13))
 (segment (start 110.2436 91.0082) (end 110.7686 91.0082) (width 0.25) (layer "F.Cu") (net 13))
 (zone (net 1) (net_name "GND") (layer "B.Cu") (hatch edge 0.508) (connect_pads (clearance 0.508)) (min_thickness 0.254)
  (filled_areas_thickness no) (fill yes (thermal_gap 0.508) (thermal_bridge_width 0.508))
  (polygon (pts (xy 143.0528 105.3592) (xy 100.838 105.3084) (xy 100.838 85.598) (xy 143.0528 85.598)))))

